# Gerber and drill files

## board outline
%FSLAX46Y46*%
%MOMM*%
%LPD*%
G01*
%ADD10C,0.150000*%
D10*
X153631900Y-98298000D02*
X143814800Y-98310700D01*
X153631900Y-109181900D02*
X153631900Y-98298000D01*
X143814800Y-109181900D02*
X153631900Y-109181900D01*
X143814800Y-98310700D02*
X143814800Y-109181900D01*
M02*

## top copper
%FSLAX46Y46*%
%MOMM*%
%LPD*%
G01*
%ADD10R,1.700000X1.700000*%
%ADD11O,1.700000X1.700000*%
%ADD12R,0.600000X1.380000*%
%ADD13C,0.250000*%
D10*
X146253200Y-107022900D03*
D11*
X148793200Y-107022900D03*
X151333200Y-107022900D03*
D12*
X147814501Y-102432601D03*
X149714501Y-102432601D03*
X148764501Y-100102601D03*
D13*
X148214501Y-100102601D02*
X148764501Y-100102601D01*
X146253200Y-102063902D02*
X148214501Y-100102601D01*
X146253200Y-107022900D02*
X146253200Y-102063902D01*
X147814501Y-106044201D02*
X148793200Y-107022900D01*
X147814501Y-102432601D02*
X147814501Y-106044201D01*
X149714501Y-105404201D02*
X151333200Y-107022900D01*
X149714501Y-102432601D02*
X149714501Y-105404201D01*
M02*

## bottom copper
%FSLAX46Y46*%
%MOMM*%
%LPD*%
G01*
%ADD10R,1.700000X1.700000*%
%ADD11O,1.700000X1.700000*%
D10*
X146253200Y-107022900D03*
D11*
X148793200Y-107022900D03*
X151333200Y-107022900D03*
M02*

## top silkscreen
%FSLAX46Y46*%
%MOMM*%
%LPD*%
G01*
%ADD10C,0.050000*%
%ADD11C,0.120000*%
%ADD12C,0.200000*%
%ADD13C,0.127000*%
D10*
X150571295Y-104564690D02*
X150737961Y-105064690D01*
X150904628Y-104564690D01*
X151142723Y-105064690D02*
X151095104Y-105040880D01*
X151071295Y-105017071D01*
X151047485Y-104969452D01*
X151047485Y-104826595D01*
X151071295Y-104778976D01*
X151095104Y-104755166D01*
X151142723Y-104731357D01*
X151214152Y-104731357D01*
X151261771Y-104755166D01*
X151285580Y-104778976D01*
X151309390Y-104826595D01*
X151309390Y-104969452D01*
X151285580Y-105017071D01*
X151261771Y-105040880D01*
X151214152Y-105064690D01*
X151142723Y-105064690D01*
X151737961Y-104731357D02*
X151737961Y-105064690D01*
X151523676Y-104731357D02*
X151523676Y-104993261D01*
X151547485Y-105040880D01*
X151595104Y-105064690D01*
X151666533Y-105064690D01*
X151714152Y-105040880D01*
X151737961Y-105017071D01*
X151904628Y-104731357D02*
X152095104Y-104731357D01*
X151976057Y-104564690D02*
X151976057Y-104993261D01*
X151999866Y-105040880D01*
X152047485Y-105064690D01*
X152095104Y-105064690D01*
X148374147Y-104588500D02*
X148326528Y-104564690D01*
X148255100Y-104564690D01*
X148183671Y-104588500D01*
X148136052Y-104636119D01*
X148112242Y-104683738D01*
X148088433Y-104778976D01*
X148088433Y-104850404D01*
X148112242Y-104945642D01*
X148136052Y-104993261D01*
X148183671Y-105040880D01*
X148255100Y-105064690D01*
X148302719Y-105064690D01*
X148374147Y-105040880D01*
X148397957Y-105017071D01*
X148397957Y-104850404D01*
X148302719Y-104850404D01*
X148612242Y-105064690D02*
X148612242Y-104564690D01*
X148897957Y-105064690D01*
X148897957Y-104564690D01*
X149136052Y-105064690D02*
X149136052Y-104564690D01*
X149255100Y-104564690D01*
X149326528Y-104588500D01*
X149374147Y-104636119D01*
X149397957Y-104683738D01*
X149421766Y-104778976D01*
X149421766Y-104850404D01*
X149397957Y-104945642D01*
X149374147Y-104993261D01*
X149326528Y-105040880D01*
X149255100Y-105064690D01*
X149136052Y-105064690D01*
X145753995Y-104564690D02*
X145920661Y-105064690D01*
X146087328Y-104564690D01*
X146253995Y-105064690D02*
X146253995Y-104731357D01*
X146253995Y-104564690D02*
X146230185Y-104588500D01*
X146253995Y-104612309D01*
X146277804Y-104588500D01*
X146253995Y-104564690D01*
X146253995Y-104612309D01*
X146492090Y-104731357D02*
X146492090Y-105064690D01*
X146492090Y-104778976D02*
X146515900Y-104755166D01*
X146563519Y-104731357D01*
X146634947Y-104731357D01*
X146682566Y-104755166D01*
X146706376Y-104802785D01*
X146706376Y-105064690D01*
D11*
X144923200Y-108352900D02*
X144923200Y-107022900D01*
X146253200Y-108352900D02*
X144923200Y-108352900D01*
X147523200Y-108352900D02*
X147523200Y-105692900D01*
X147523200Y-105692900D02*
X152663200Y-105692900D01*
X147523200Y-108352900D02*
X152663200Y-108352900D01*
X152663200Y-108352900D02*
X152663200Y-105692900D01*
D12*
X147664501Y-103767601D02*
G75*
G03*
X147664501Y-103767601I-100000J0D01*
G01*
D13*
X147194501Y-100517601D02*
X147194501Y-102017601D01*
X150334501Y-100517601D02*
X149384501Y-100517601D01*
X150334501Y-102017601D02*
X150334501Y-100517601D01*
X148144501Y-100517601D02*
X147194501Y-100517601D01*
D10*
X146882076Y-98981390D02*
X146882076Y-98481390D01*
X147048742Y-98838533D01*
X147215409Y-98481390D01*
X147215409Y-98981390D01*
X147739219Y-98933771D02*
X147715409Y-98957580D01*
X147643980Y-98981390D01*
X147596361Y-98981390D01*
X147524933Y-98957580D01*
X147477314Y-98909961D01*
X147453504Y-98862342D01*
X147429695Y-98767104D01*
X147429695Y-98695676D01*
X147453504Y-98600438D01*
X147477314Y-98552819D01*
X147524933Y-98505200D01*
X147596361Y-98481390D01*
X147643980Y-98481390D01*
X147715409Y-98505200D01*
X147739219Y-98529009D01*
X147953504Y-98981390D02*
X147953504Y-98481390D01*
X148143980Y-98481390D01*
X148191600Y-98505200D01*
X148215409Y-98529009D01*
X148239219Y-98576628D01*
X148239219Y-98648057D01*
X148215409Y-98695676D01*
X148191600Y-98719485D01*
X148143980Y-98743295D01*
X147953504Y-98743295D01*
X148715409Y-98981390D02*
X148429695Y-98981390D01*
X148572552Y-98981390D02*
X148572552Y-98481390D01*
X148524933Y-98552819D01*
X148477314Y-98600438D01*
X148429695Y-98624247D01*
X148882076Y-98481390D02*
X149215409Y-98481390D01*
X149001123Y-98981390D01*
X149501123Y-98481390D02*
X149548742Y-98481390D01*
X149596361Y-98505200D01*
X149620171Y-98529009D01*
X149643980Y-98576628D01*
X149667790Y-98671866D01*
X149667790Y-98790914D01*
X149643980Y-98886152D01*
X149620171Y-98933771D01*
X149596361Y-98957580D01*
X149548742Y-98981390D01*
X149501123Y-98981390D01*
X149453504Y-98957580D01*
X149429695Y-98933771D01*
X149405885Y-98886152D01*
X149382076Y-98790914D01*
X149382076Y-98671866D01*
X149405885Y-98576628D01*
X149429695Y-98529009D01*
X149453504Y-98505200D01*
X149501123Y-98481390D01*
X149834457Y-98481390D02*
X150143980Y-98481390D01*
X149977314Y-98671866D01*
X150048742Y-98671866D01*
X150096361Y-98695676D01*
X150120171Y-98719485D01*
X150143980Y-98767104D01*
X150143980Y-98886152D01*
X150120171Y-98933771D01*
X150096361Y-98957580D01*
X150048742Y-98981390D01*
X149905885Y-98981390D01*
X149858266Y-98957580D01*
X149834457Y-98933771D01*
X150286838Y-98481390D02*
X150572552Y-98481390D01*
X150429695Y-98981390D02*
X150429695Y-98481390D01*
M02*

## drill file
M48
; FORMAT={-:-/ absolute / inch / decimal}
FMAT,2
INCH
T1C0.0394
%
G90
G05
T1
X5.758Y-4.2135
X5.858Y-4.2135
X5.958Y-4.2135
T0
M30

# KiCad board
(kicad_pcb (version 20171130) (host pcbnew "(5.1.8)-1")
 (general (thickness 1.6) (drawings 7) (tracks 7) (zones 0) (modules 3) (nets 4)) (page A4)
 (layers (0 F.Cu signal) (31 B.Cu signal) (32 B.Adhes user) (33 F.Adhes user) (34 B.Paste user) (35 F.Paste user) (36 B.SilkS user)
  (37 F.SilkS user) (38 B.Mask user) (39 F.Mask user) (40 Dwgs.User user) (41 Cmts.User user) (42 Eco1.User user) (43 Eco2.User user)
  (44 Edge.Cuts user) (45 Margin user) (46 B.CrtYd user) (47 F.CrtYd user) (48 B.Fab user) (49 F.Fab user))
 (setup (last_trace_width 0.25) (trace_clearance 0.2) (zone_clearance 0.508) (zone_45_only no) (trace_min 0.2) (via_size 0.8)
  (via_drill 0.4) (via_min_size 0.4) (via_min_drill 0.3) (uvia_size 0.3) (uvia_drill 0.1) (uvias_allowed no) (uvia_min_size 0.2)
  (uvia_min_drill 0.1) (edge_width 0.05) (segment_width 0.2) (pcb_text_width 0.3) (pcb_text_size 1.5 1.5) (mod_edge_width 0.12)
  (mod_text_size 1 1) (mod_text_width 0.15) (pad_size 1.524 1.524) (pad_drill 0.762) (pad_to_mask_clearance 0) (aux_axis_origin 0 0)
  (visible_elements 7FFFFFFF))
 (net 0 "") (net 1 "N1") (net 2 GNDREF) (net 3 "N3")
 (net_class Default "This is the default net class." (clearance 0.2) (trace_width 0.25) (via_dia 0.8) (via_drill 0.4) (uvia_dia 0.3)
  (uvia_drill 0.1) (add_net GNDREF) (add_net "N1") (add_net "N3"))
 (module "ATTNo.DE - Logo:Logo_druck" (layer B.Cu) (at 148.8694 103.3272 180)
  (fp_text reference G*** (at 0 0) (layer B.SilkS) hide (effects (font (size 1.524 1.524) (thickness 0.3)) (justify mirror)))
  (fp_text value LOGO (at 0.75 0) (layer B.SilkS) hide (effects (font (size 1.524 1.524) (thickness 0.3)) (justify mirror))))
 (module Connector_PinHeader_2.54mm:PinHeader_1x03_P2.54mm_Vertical (layer F.Cu) (at 146.2532 107.0229 90)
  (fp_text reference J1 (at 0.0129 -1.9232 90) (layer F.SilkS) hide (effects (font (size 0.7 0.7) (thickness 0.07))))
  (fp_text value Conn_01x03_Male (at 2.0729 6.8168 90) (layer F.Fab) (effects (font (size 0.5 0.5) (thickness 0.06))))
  (fp_line (start -1.33 -1.33) (end 0 -1.33) (layer F.SilkS) (width 0.12))
  (fp_line (start -1.33 0) (end -1.33 -1.33) (layer F.SilkS) (width 0.12))
  (fp_line (start -1.33 1.27) (end 1.33 1.27) (layer F.SilkS) (width 0.12))
  (fp_line (start 1.33 1.27) (end 1.33 6.41) (layer F.SilkS) (width 0.12))
  (fp_line (start -1.33 1.27) (end -1.33 6.41) (layer F.SilkS) (width 0.12))
  (fp_line (start -1.33 6.41) (end 1.33 6.41) (layer F.SilkS) (width 0.12))
  (pad 1 thru_hole rect (at 0 0 90) (size 1.7 1.7) (drill 1) (layers *.Cu *.Mask) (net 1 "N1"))
  (pad 2 thru_hole oval (at 0 2.54 90) (size 1.7 1.7) (drill 1) (layers *.Cu *.Mask) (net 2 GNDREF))
  (pad 3 thru_hole oval (at 0 5.08 90) (size 1.7 1.7) (drill 1) (layers *.Cu *.Mask) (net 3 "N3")))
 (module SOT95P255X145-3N (layer F.Cu) (at 148.764501 101.267601 90)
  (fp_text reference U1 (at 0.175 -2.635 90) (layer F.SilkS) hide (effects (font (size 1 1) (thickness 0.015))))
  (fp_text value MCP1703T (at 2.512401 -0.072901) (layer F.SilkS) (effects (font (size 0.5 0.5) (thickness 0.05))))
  (fp_circle (center -2.5 -1.2) (end -2.4 -1.2) (layer F.SilkS) (width 0.2))
  (fp_line (start 0.75 -1.57) (end -0.75 -1.57) (layer F.SilkS) (width 0.127))
  (fp_line (start 0.75 1.57) (end 0.75 0.62) (layer F.SilkS) (width 0.127))
  (fp_line (start -0.75 1.57) (end 0.75 1.57) (layer F.SilkS) (width 0.127))
  (fp_line (start 0.75 -0.62) (end 0.75 -1.57) (layer F.SilkS) (width 0.127))
  (pad 1 smd rect (at -1.165 -0.95 90) (size 1.38 0.6) (layers F.Cu F.Paste F.Mask) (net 2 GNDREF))
  (pad 2 smd rect (at -1.165 0.95 90) (size 1.38 0.6) (layers F.Cu F.Paste F.Mask) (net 3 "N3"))
  (pad 3 smd rect (at 1.165 0 90) (size 1.38 0.6) (layers F.Cu F.Paste F.Mask) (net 1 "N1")))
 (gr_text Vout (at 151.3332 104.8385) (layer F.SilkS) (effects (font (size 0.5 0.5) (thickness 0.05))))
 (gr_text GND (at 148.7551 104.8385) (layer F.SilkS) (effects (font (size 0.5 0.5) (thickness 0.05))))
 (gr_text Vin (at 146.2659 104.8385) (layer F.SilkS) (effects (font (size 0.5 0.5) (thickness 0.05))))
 (gr_line (start 153.6319 98.298) (end 143.8148 98.3107) (layer Edge.Cuts) (width 0.15))
 (gr_line (start 153.6319 109.1819) (end 153.6319 98.298) (layer Edge.Cuts) (width 0.15))
 (gr_line (start 143.8148 109.1819) (end 153.6319 109.1819) (layer Edge.Cuts) (width 0.15))
 (gr_line (start 143.8148 98.3107) (end 143.8148 109.1819) (layer Edge.Cuts) (width 0.15))
 (segment (start 148.214501 100.102601) (end 148.764501 100.102601) (width 0.25) (layer F.Cu) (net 1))
 (segment (start 146.2532 102.063902) (end 148.214501 100.102601) (width 0.25) (layer F.Cu) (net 1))
 (segment (start 146.2532 107.0229) (end 146.2532 102.063902) (width 0.25) (layer F.Cu) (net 1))
 (segment (start 147.814501 106.044201) (end 148.7932 107.0229) (width 0.25) (layer F.Cu) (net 2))
 (segment (start 147.814501 102.432601) (end 147.814501 106.044201) (width 0.25) (layer F.Cu) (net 2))
 (segment (start 149.714501 105.404201) (end 151.3332 107.0229) (width 0.25) (layer F.Cu) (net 3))
 (segment (start 149.714501 102.432601) (end 149.714501 105.404201) (width 0.25) (layer F.Cu) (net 3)))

